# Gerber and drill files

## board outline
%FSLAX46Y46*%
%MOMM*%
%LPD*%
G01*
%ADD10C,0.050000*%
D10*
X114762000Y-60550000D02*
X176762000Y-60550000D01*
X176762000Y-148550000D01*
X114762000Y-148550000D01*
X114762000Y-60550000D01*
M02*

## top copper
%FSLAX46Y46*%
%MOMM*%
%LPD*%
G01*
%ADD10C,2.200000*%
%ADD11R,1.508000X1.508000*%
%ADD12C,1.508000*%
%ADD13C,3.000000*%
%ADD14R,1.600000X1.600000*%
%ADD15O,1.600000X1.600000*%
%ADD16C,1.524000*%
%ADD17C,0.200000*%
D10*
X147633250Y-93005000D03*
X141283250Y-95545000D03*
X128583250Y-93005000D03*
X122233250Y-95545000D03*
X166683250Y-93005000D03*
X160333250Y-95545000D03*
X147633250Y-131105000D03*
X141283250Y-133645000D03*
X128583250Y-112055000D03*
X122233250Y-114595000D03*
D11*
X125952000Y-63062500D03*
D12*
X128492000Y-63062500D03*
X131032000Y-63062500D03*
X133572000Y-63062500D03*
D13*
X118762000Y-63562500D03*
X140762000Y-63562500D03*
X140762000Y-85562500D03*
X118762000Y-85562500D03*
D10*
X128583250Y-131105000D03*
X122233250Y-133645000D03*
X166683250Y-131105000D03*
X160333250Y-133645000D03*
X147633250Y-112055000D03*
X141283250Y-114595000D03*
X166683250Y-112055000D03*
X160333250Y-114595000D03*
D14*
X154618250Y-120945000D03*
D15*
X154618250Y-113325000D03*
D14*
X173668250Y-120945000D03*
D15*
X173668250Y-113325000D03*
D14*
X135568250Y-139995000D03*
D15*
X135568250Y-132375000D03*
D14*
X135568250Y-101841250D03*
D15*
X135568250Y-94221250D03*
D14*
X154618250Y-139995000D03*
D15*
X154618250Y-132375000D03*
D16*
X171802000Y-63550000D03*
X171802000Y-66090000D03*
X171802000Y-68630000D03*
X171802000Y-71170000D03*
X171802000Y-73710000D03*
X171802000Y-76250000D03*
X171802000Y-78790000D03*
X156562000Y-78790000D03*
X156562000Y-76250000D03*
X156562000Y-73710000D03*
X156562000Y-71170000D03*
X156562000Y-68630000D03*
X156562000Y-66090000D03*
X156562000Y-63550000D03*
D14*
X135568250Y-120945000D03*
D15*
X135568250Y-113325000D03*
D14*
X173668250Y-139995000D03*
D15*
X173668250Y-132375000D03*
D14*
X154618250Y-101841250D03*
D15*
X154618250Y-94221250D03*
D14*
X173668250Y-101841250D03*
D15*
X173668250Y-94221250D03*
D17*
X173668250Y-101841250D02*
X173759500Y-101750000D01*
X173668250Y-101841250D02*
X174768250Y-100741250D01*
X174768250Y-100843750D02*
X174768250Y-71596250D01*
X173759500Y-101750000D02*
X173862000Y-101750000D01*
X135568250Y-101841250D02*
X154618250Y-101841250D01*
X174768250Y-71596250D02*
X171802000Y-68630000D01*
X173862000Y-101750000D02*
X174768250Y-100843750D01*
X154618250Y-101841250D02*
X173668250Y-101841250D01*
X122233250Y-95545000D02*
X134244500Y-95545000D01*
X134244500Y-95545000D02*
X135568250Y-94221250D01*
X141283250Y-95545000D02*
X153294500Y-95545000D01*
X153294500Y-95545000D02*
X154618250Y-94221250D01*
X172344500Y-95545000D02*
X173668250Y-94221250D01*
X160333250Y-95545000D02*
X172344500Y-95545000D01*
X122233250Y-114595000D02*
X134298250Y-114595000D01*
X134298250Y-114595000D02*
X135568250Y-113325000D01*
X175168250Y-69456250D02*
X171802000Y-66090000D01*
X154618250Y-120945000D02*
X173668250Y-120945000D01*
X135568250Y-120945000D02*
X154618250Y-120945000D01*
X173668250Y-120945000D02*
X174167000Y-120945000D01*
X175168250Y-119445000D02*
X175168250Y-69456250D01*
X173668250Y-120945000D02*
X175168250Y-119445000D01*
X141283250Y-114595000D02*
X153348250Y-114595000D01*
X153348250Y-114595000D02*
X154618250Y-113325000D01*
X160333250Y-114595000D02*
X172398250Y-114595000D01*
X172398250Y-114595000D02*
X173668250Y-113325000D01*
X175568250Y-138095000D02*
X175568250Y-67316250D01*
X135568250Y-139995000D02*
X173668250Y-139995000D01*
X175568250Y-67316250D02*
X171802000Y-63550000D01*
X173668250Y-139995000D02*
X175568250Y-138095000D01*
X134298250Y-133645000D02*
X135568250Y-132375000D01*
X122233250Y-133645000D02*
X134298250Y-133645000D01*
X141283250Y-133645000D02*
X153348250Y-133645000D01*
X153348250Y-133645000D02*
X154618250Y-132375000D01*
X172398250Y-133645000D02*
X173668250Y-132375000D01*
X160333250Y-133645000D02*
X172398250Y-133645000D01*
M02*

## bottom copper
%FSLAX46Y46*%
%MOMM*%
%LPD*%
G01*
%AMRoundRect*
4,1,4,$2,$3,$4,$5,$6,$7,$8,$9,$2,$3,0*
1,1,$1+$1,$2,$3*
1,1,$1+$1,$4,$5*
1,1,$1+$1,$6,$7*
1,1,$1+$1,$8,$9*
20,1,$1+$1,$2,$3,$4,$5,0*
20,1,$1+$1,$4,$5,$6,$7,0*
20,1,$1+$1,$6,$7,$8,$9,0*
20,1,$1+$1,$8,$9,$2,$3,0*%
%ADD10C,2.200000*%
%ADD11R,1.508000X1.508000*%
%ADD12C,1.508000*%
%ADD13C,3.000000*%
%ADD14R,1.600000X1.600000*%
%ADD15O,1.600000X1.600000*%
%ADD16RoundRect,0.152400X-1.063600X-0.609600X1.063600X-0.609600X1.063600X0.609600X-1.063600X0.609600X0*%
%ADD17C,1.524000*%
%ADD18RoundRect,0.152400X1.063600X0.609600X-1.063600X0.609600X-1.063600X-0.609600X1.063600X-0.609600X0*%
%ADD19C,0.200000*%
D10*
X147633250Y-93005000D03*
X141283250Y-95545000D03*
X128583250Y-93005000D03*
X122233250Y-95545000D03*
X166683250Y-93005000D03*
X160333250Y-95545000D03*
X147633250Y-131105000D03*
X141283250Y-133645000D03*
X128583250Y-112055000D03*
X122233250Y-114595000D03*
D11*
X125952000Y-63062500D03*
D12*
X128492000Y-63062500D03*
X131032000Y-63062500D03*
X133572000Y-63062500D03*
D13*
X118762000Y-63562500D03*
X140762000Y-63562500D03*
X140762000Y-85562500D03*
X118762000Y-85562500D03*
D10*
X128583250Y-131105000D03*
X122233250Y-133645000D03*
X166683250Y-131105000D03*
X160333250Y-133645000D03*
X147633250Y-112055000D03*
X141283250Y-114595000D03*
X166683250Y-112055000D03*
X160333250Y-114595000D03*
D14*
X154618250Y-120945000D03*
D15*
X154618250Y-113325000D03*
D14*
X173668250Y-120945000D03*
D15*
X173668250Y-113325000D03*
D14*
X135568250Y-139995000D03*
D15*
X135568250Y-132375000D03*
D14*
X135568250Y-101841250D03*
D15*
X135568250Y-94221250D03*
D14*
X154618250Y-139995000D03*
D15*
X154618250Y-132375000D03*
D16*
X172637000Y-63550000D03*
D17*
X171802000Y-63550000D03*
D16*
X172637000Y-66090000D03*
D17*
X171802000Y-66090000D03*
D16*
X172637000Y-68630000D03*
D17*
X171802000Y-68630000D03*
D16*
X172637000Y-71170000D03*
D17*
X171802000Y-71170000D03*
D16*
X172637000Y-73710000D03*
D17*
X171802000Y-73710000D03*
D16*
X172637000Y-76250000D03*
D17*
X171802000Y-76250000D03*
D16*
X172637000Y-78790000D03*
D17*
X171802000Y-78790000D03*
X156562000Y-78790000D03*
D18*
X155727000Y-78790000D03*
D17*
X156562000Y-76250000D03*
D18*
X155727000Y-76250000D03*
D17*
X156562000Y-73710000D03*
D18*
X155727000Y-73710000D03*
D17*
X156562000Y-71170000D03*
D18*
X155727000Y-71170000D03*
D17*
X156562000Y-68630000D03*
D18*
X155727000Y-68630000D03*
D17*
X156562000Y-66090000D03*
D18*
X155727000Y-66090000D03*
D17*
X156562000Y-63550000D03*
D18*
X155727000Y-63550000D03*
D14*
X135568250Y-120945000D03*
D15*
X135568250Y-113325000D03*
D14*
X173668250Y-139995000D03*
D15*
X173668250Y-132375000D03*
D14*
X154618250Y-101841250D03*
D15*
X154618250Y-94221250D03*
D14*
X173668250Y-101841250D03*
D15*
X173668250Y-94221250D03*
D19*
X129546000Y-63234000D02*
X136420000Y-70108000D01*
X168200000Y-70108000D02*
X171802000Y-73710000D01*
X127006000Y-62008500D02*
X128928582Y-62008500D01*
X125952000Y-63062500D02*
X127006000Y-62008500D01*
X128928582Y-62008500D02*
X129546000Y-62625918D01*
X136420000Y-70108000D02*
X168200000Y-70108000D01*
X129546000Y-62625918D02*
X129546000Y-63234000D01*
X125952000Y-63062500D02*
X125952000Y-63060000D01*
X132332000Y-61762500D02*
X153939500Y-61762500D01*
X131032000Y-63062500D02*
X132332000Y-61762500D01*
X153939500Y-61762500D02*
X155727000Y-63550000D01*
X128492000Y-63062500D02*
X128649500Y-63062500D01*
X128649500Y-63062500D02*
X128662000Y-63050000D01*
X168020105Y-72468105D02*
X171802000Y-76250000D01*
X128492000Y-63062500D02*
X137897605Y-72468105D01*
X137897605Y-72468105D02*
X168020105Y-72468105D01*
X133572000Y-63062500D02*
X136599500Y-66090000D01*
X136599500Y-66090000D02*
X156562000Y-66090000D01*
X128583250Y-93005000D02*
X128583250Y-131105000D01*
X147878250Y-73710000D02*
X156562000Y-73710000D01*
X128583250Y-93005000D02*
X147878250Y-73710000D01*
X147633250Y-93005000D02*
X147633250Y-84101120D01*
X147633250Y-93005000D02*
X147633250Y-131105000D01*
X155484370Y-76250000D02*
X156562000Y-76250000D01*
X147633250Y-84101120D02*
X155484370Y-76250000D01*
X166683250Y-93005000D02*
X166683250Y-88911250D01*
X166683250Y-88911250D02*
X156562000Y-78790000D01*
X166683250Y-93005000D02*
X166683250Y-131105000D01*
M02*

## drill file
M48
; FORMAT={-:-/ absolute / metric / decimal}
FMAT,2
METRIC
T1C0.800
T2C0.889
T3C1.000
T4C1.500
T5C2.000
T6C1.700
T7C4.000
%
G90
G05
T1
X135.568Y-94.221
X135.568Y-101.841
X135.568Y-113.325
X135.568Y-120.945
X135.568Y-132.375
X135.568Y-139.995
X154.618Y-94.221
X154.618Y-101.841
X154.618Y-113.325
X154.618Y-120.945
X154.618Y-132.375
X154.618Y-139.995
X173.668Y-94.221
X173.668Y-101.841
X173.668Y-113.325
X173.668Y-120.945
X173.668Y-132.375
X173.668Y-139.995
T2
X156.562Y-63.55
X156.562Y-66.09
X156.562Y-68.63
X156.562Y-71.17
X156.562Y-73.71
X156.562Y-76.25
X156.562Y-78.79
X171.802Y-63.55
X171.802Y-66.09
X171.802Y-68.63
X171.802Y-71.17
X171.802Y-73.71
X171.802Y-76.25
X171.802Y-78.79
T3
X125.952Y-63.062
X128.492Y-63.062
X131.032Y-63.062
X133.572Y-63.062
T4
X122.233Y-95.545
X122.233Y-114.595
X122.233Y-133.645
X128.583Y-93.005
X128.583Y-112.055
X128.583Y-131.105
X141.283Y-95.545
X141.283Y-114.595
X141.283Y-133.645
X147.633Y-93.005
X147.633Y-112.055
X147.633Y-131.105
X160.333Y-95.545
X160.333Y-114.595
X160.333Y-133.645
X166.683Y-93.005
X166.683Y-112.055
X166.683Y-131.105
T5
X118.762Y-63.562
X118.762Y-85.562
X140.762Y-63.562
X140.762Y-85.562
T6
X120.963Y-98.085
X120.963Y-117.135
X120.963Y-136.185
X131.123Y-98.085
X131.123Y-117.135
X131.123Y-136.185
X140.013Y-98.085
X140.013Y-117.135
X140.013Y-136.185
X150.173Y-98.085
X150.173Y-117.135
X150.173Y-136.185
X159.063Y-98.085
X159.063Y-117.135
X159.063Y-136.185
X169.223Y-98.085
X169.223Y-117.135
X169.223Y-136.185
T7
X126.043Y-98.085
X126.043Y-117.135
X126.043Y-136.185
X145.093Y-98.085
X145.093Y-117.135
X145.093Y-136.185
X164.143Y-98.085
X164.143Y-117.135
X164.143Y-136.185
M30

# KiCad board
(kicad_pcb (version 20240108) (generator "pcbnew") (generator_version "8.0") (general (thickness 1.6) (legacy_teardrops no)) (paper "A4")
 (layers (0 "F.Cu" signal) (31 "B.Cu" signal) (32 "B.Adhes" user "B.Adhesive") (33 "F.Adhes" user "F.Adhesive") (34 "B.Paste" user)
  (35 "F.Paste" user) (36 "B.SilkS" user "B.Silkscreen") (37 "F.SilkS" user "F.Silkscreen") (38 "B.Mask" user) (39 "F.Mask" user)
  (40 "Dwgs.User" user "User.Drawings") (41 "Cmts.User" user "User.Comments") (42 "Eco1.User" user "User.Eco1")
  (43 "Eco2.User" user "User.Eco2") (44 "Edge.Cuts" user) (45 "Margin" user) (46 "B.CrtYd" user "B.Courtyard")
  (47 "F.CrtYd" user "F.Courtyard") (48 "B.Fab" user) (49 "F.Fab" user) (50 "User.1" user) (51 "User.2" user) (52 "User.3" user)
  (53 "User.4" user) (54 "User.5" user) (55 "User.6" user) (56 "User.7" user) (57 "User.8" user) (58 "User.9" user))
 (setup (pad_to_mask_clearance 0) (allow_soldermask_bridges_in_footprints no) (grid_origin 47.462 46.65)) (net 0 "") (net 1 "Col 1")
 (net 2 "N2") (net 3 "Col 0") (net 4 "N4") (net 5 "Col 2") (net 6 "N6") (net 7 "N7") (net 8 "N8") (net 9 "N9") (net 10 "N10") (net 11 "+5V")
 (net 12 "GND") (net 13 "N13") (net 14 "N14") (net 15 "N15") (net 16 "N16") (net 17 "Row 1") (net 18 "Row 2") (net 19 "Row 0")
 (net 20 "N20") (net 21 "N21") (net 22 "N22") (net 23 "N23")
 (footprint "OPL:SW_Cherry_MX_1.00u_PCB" (layer "F.Cu") (at 147.63325 93.005)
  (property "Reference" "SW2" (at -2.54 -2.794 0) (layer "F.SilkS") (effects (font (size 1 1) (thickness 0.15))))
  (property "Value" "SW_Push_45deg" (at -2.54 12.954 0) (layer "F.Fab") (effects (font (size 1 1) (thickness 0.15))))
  (pad "" np_thru_hole circle (at -7.62 5.08) (size 1.7 1.7) (drill 1.7) (layers "*.Cu" "*.Mask"))
  (pad "" np_thru_hole circle (at -2.54 5.08) (size 4 4) (drill 4) (layers "*.Cu" "*.Mask"))
  (pad "" np_thru_hole circle (at 2.54 5.08) (size 1.7 1.7) (drill 1.7) (layers "*.Cu" "*.Mask"))
  (pad "1" thru_hole circle (at 0 0) (size 2.2 2.2) (drill 1.5) (layers "*.Cu" "*.Mask") (remove_unused_layers no) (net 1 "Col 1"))
  (pad "2" thru_hole circle (at -6.35 2.54) (size 2.2 2.2) (drill 1.5) (layers "*.Cu" "*.Mask") (remove_unused_layers no) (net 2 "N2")))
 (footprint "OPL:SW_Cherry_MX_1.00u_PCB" (layer "F.Cu") (at 128.58325 93.005)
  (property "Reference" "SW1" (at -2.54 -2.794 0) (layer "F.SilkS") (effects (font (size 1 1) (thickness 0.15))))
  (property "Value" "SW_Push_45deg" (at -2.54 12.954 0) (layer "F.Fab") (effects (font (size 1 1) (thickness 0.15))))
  (pad "" np_thru_hole circle (at -7.62 5.08) (size 1.7 1.7) (drill 1.7) (layers "*.Cu" "*.Mask"))
  (pad "" np_thru_hole circle (at -2.54 5.08) (size 4 4) (drill 4) (layers "*.Cu" "*.Mask"))
  (pad "" np_thru_hole circle (at 2.54 5.08) (size 1.7 1.7) (drill 1.7) (layers "*.Cu" "*.Mask"))
  (pad "1" thru_hole circle (at 0 0) (size 2.2 2.2) (drill 1.5) (layers "*.Cu" "*.Mask") (remove_unused_layers no) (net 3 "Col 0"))
  (pad "2" thru_hole circle (at -6.35 2.54) (size 2.2 2.2) (drill 1.5) (layers "*.Cu" "*.Mask") (remove_unused_layers no) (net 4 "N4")))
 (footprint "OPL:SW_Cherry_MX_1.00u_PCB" (layer "F.Cu") (at 166.68325 93.005)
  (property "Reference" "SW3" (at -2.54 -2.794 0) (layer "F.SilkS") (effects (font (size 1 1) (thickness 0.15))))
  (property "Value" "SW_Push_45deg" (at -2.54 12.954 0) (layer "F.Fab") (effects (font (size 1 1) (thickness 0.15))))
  (pad "" np_thru_hole circle (at -7.62 5.08) (size 1.7 1.7) (drill 1.7) (layers "*.Cu" "*.Mask"))
  (pad "" np_thru_hole circle (at -2.54 5.08) (size 4 4) (drill 4) (layers "*.Cu" "*.Mask"))
  (pad "" np_thru_hole circle (at 2.54 5.08) (size 1.7 1.7) (drill 1.7) (layers "*.Cu" "*.Mask"))
  (pad "1" thru_hole circle (at 0 0) (size 2.2 2.2) (drill 1.5) (layers "*.Cu" "*.Mask") (remove_unused_layers no) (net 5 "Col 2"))
  (pad "2" thru_hole circle (at -6.35 2.54) (size 2.2 2.2) (drill 1.5) (layers "*.Cu" "*.Mask") (remove_unused_layers no) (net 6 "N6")))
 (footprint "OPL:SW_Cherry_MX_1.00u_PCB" (layer "F.Cu") (at 147.63325 131.105)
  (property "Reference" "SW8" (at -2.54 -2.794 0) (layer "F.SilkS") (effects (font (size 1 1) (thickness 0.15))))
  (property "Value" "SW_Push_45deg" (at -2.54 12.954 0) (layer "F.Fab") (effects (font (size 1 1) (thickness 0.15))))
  (pad "" np_thru_hole circle (at -7.62 5.08) (size 1.7 1.7) (drill 1.7) (layers "*.Cu" "*.Mask"))
  (pad "" np_thru_hole circle (at -2.54 5.08) (size 4 4) (drill 4) (layers "*.Cu" "*.Mask"))
  (pad "" np_thru_hole circle (at 2.54 5.08) (size 1.7 1.7) (drill 1.7) (layers "*.Cu" "*.Mask"))
  (pad "1" thru_hole circle (at 0 0) (size 2.2 2.2) (drill 1.5) (layers "*.Cu" "*.Mask") (remove_unused_layers no) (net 1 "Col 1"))
  (pad "2" thru_hole circle (at -6.35 2.54) (size 2.2 2.2) (drill 1.5) (layers "*.Cu" "*.Mask") (remove_unused_layers no) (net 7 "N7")))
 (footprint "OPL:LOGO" (layer "F.Cu") (at 161.562 84.85)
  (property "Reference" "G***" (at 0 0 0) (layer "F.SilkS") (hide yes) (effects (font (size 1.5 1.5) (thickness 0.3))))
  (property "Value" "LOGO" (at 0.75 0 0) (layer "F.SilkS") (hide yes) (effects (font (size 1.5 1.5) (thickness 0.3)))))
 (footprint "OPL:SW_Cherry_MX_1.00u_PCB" (layer "F.Cu") (at 128.58325 112.055)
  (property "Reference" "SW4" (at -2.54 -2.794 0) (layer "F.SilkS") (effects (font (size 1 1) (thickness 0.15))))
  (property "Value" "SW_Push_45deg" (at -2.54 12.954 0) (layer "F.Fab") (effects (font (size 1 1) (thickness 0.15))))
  (pad "" np_thru_hole circle (at -7.62 5.08) (size 1.7 1.7) (drill 1.7) (layers "*.Cu" "*.Mask"))
  (pad "" np_thru_hole circle (at -2.54 5.08) (size 4 4) (drill 4) (layers "*.Cu" "*.Mask"))
  (pad "" np_thru_hole circle (at 2.54 5.08) (size 1.7 1.7) (drill 1.7) (layers "*.Cu" "*.Mask"))
  (pad "1" thru_hole circle (at 0 0) (size 2.2 2.2) (drill 1.5) (layers "*.Cu" "*.Mask") (remove_unused_layers no) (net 3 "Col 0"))
  (pad "2" thru_hole circle (at -6.35 2.54) (size 2.2 2.2) (drill 1.5) (layers "*.Cu" "*.Mask") (remove_unused_layers no) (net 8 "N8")))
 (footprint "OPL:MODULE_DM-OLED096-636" (layer "F.Cu") (at 129.762 74.5625)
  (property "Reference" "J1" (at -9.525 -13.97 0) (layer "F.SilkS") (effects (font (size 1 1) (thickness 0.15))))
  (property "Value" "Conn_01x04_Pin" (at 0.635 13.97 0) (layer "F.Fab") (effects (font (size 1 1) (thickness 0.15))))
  (pad "1" thru_hole rect (at -3.81 -11.5) (size 1.508 1.508) (drill 1) (layers "*.Cu" "*.Mask") (remove_unused_layers no) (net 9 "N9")
   (solder_mask_margin 0.102))
  (pad "2" thru_hole circle (at -1.27 -11.5) (size 1.508 1.508) (drill 1) (layers "*.Cu" "*.Mask") (remove_unused_layers no) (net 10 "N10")
   (solder_mask_margin 0.102))
  (pad "3" thru_hole circle (at 1.27 -11.5) (size 1.508 1.508) (drill 1) (layers "*.Cu" "*.Mask") (remove_unused_layers no) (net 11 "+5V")
   (solder_mask_margin 0.102))
  (pad "4" thru_hole circle (at 3.81 -11.5) (size 1.508 1.508) (drill 1) (layers "*.Cu" "*.Mask") (remove_unused_layers no) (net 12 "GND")
   (solder_mask_margin 0.102))
  (pad "S1" thru_hole circle (at -11 -11) (size 3 3) (drill 2) (layers "*.Cu" "*.Mask") (remove_unused_layers no) (solder_mask_margin 0.102))
  (pad "S2" thru_hole circle (at 11 -11) (size 3 3) (drill 2) (layers "*.Cu" "*.Mask") (remove_unused_layers no) (solder_mask_margin 0.102))
  (pad "S3" thru_hole circle (at 11 11) (size 3 3) (drill 2) (layers "*.Cu" "*.Mask") (remove_unused_layers no) (solder_mask_margin 0.102))
  (pad "S4" thru_hole circle (at -11 11) (size 3 3) (drill 2) (layers "*.Cu" "*.Mask") (remove_unused_layers no) (solder_mask_margin 0.102)))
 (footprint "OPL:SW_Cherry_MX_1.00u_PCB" (layer "F.Cu") (at 128.58325 131.105)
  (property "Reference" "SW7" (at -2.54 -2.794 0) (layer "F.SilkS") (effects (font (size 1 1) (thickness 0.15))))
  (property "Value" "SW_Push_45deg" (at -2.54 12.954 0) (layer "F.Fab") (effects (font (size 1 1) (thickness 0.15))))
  (pad "" np_thru_hole circle (at -7.62 5.08) (size 1.7 1.7) (drill 1.7) (layers "*.Cu" "*.Mask"))
  (pad "" np_thru_hole circle (at -2.54 5.08) (size 4 4) (drill 4) (layers "*.Cu" "*.Mask"))
  (pad "" np_thru_hole circle (at 2.54 5.08) (size 1.7 1.7) (drill 1.7) (layers "*.Cu" "*.Mask"))
  (pad "1" thru_hole circle (at 0 0) (size 2.2 2.2) (drill 1.5) (layers "*.Cu" "*.Mask") (remove_unused_layers no) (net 3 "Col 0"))
  (pad "2" thru_hole circle (at -6.35 2.54) (size 2.2 2.2) (drill 1.5) (layers "*.Cu" "*.Mask") (remove_unused_layers no) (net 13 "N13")))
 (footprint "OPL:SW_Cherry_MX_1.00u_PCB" (layer "F.Cu") (at 166.68325 131.105)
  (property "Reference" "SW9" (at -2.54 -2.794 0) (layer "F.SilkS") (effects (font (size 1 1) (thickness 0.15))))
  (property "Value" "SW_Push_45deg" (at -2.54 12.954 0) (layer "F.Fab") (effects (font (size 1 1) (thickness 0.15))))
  (pad "" np_thru_hole circle (at -7.62 5.08) (size 1.7 1.7) (drill 1.7) (layers "*.Cu" "*.Mask"))
  (pad "" np_thru_hole circle (at -2.54 5.08) (size 4 4) (drill 4) (layers "*.Cu" "*.Mask"))
  (pad "" np_thru_hole circle (at 2.54 5.08) (size 1.7 1.7) (drill 1.7) (layers "*.Cu" "*.Mask"))
  (pad "1" thru_hole circle (at 0 0) (size 2.2 2.2) (drill 1.5) (layers "*.Cu" "*.Mask") (remove_unused_layers no) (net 5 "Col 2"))
  (pad "2" thru_hole circle (at -6.35 2.54) (size 2.2 2.2) (drill 1.5) (layers "*.Cu" "*.Mask") (remove_unused_layers no) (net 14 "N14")))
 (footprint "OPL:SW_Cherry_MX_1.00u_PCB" (layer "F.Cu") (at 147.63325 112.055)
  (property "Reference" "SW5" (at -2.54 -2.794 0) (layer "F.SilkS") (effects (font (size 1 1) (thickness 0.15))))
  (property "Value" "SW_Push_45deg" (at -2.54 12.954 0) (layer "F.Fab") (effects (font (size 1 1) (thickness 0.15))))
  (pad "" np_thru_hole circle (at -7.62 5.08) (size 1.7 1.7) (drill 1.7) (layers "*.Cu" "*.Mask"))
  (pad "" np_thru_hole circle (at -2.54 5.08) (size 4 4) (drill 4) (layers "*.Cu" "*.Mask"))
  (pad "" np_thru_hole circle (at 2.54 5.08) (size 1.7 1.7) (drill 1.7) (layers "*.Cu" "*.Mask"))
  (pad "1" thru_hole circle (at 0 0) (size 2.2 2.2) (drill 1.5) (layers "*.Cu" "*.Mask") (remove_unused_layers no) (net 1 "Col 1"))
  (pad "2" thru_hole circle (at -6.35 2.54) (size 2.2 2.2) (drill 1.5) (layers "*.Cu" "*.Mask") (remove_unused_layers no) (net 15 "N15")))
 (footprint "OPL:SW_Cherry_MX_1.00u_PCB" (layer "F.Cu") (at 166.68325 112.055)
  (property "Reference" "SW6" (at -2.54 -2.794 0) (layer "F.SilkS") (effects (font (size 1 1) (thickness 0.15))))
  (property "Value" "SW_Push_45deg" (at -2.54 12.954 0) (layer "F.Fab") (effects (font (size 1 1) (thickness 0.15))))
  (pad "" np_thru_hole circle (at -7.62 5.08) (size 1.7 1.7) (drill 1.7) (layers "*.Cu" "*.Mask"))
  (pad "" np_thru_hole circle (at -2.54 5.08) (size 4 4) (drill 4) (layers "*.Cu" "*.Mask"))
  (pad "" np_thru_hole circle (at 2.54 5.08) (size 1.7 1.7) (drill 1.7) (layers "*.Cu" "*.Mask"))
  (pad "1" thru_hole circle (at 0 0) (size 2.2 2.2) (drill 1.5) (layers "*.Cu" "*.Mask") (remove_unused_layers no) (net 5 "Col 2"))
  (pad "2" thru_hole circle (at -6.35 2.54) (size 2.2 2.2) (drill 1.5) (layers "*.Cu" "*.Mask") (remove_unused_layers no) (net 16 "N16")))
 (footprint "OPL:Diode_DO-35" (layer "B.Cu") (at 154.61825 120.945 90)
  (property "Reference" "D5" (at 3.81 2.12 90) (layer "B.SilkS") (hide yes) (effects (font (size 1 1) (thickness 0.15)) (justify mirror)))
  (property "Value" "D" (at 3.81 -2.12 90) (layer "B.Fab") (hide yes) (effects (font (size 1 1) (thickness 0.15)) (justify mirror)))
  (pad "1" thru_hole rect (at 0 0 90) (size 1.6 1.6) (drill 0.8) (layers "*.Cu" "*.Mask") (remove_unused_layers no) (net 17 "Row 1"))
  (pad "2" thru_hole oval (at 7.62 0 90) (size 1.6 1.6) (drill 0.8) (layers "*.Cu" "*.Mask") (remove_unused_layers no) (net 15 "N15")))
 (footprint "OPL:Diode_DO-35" (layer "B.Cu") (at 173.66825 120.945 90)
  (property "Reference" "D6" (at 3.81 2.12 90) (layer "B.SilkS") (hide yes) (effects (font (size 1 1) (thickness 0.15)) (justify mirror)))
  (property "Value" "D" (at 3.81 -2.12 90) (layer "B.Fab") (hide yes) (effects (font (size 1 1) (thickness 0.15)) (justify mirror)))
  (pad "1" thru_hole rect (at 0 0 90) (size 1.6 1.6) (drill 0.8) (layers "*.Cu" "*.Mask") (remove_unused_layers no) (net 17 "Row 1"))
  (pad "2" thru_hole oval (at 7.62 0 90) (size 1.6 1.6) (drill 0.8) (layers "*.Cu" "*.Mask") (remove_unused_layers no) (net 16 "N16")))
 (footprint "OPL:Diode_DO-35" (layer "B.Cu") (at 135.56825 139.995 90)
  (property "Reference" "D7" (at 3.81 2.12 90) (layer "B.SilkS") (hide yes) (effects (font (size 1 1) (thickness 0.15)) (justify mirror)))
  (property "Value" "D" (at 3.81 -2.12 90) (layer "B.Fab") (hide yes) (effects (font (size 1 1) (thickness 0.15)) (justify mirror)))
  (pad "1" thru_hole rect (at 0 0 90) (size 1.6 1.6) (drill 0.8) (layers "*.Cu" "*.Mask") (remove_unused_layers no) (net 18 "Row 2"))
  (pad "2" thru_hole oval (at 7.62 0 90) (size 1.6 1.6) (drill 0.8) (layers "*.Cu" "*.Mask") (remove_unused_layers no) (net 13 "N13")))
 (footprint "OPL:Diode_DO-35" (layer "B.Cu") (at 135.56825 101.84125 90)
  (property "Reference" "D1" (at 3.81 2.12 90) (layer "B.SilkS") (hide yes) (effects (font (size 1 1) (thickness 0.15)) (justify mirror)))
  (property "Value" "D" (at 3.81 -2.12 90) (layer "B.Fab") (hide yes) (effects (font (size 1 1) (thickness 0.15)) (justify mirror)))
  (pad "1" thru_hole rect (at 0 0 90) (size 1.6 1.6) (drill 0.8) (layers "*.Cu" "*.Mask") (remove_unused_layers no) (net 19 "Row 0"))
  (pad "2" thru_hole oval (at 7.62 0 90) (size 1.6 1.6) (drill 0.8) (layers "*.Cu" "*.Mask") (remove_unused_layers no) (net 4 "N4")))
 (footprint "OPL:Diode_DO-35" (layer "B.Cu") (at 154.61825 139.995 90)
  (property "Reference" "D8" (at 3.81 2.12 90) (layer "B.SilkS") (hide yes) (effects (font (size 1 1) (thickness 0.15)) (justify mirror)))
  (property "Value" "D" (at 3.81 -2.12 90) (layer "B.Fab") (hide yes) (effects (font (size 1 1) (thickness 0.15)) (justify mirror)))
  (pad "1" thru_hole rect (at 0 0 90) (size 1.6 1.6) (drill 0.8) (layers "*.Cu" "*.Mask") (remove_unused_layers no) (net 18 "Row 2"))
  (pad "2" thru_hole oval (at 7.62 0 90) (size 1.6 1.6) (drill 0.8) (layers "*.Cu" "*.Mask") (remove_unused_layers no) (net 7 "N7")))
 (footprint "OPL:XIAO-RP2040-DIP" (layer "B.Cu") (at 164.182 71.17 180)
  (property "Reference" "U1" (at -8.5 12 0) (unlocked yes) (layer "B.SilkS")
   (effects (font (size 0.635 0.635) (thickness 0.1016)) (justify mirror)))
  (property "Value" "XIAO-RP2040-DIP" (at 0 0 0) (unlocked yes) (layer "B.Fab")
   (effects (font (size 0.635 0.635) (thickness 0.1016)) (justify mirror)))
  (pad "1" smd roundrect (at -8.455 7.62) (size 2.432 1.524) (layers "B.Cu" "B.Mask") (roundrect_rratio 0.1) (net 18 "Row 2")
   (thermal_bridge_angle 45))
  (pad "1" thru_hole circle (at -7.62 7.62) (size 1.524 1.524) (drill 0.889) (layers "*.Cu" "*.Mask") (remove_unused_layers no)
   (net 18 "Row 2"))
  (pad "2" smd roundrect (at -8.455 5.08) (size 2.432 1.524) (layers "B.Cu" "B.Mask") (roundrect_rratio 0.1) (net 17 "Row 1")
   (thermal_bridge_angle 45))
  (pad "2" thru_hole circle (at -7.62 5.08) (size 1.524 1.524) (drill 0.889) (layers "*.Cu" "*.Mask") (remove_unused_layers no)
   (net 17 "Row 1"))
  (pad "3" smd roundrect (at -8.455 2.54) (size 2.432 1.524) (layers "B.Cu" "B.Mask") (roundrect_rratio 0.1) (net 19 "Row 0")
   (thermal_bridge_angle 45))
  (pad "3" thru_hole circle (at -7.62 2.54) (size 1.524 1.524) (drill 0.889) (layers "*.Cu" "*.Mask") (remove_unused_layers no)
   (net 19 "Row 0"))
  (pad "4" smd roundrect (at -8.455 0) (size 2.432 1.524) (layers "B.Cu" "B.Mask") (roundrect_rratio 0.1) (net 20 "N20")
   (thermal_bridge_angle 45))
  (pad "4" thru_hole circle (at -7.62 0) (size 1.524 1.524) (drill 0.889) (layers "*.Cu" "*.Mask") (remove_unused_layers no) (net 20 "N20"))
  (pad "5" smd roundrect (at -8.455 -2.54) (size 2.432 1.524) (layers "B.Cu" "B.Mask") (roundrect_rratio 0.1) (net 9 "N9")
   (thermal_bridge_angle 45))
  (pad "5" thru_hole circle (at -7.62 -2.54) (size 1.524 1.524) (drill 0.889) (layers "*.Cu" "*.Mask") (remove_unused_layers no)
   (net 9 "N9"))
  (pad "6" smd roundrect (at -8.455 -5.08) (size 2.432 1.524) (layers "B.Cu" "B.Mask") (roundrect_rratio 0.1) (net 10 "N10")
   (thermal_bridge_angle 45))
  (pad "6" thru_hole circle (at -7.62 -5.08) (size 1.524 1.524) (drill 0.889) (layers "*.Cu" "*.Mask") (remove_unused_layers no)
   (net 10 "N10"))
  (pad "7" smd roundrect (at -8.455 -7.62) (size 2.432 1.524) (layers "B.Cu" "B.Mask") (roundrect_rratio 0.1) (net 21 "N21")
   (thermal_bridge_angle 45))
  (pad "7" thru_hole circle (at -7.62 -7.62) (size 1.524 1.524) (drill 0.889) (layers "*.Cu" "*.Mask") (remove_unused_layers no)
   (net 21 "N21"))
  (pad "8" thru_hole circle (at 7.62 -7.62 180) (size 1.524 1.524) (drill 0.889) (layers "*.Cu" "*.Mask") (remove_unused_layers no)
   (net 5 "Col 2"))
  (pad "8" smd roundrect (at 8.455 -7.62 180) (size 2.432 1.524) (layers "B.Cu" "B.Mask") (roundrect_rratio 0.1) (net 5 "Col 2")
   (thermal_bridge_angle 45))
  (pad "9" thru_hole circle (at 7.62 -5.08 180) (size 1.524 1.524) (drill 0.889) (layers "*.Cu" "*.Mask") (remove_unused_layers no)
   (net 1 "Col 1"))
  (pad "9" smd roundrect (at 8.455 -5.08 180) (size 2.432 1.524) (layers "B.Cu" "B.Mask") (roundrect_rratio 0.1) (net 1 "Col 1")
   (thermal_bridge_angle 45))
  (pad "10" thru_hole circle (at 7.62 -2.54 180) (size 1.524 1.524) (drill 0.889) (layers "*.Cu" "*.Mask") (remove_unused_layers no)
   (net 3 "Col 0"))
  (pad "10" smd roundrect (at 8.455 -2.54 180) (size 2.432 1.524) (layers "B.Cu" "B.Mask") (roundrect_rratio 0.1) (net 3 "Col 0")
   (thermal_bridge_angle 45))
  (pad "11" thru_hole circle (at 7.62 0 180) (size 1.524 1.524) (drill 0.889) (layers "*.Cu" "*.Mask") (remove_unused_layers no)
   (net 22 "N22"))
  (pad "11" smd roundrect (at 8.455 0 180) (size 2.432 1.524) (layers "B.Cu" "B.Mask") (roundrect_rratio 0.1) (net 22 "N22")
   (thermal_bridge_angle 45))
  (pad "12" thru_hole circle (at 7.62 2.54 180) (size 1.524 1.524) (drill 0.889) (layers "*.Cu" "*.Mask") (remove_unused_layers no)
   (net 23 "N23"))
  (pad "12" smd roundrect (at 8.455 2.54 180) (size 2.432 1.524) (layers "B.Cu" "B.Mask") (roundrect_rratio 0.1) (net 23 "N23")
   (thermal_bridge_angle 45))
  (pad "13" thru_hole circle (at 7.62 5.08 180) (size 1.524 1.524) (drill 0.889) (layers "*.Cu" "*.Mask") (remove_unused_layers no)
   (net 12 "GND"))
  (pad "13" smd roundrect (at 8.455 5.08 180) (size 2.432 1.524) (layers "B.Cu" "B.Mask") (roundrect_rratio 0.1) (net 12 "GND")
   (thermal_bridge_angle 45))
  (pad "14" thru_hole circle (at 7.62 7.62 180) (size 1.524 1.524) (drill 0.889) (layers "*.Cu" "*.Mask") (remove_unused_layers no)
   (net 11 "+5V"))
  (pad "14" smd roundrect (at 8.455 7.62 180) (size 2.432 1.524) (layers "B.Cu" "B.Mask") (roundrect_rratio 0.1) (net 11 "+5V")
   (thermal_bridge_angle 45)))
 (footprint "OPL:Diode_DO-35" (layer "B.Cu") (at 135.56825 120.945 90)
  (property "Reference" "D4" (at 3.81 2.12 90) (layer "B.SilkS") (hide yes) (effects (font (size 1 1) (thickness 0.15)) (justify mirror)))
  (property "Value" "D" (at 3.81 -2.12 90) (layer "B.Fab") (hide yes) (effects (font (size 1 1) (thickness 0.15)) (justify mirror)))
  (pad "1" thru_hole rect (at 0 0 90) (size 1.6 1.6) (drill 0.8) (layers "*.Cu" "*.Mask") (remove_unused_layers no) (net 17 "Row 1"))
  (pad "2" thru_hole oval (at 7.62 0 90) (size 1.6 1.6) (drill 0.8) (layers "*.Cu" "*.Mask") (remove_unused_layers no) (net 8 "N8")))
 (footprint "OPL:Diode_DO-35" (layer "B.Cu") (at 173.66825 139.995 90)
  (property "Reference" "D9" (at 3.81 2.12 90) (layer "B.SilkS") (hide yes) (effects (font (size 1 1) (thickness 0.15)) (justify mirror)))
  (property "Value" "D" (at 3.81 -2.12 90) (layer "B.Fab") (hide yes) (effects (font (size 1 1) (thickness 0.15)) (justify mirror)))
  (pad "1" thru_hole rect (at 0 0 90) (size 1.6 1.6) (drill 0.8) (layers "*.Cu" "*.Mask") (remove_unused_layers no) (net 18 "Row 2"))
  (pad "2" thru_hole oval (at 7.62 0 90) (size 1.6 1.6) (drill 0.8) (layers "*.Cu" "*.Mask") (remove_unused_layers no) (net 14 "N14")))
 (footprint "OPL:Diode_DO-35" (layer "B.Cu") (at 154.61825 101.84125 90)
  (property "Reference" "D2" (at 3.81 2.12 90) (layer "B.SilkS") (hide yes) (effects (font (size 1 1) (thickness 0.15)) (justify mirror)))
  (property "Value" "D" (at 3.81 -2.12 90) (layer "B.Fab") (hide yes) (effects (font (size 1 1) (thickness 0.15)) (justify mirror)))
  (pad "1" thru_hole rect (at 0 0 90) (size 1.6 1.6) (drill 0.8) (layers "*.Cu" "*.Mask") (remove_unused_layers no) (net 19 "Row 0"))
  (pad "2" thru_hole oval (at 7.62 0 90) (size 1.6 1.6) (drill 0.8) (layers "*.Cu" "*.Mask") (remove_unused_layers no) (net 2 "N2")))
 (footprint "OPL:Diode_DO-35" (layer "B.Cu") (at 173.66825 101.84125 90)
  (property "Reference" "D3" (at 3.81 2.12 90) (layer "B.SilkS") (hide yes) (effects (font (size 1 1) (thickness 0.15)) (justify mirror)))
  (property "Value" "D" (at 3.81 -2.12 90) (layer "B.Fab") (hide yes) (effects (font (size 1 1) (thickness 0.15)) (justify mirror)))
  (pad "1" thru_hole rect (at 0 0 90) (size 1.6 1.6) (drill 0.8) (layers "*.Cu" "*.Mask") (remove_unused_layers no) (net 19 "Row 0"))
  (pad "2" thru_hole oval (at 7.62 0 90) (size 1.6 1.6) (drill 0.8) (layers "*.Cu" "*.Mask") (remove_unused_layers no) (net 6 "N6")))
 (gr_rect (start 114.762 60.55) (end 176.762 148.55) (stroke (width 0.05) (type default)) (fill none) (layer "Edge.Cuts"))
 (segment (start 173.66825 101.84125) (end 173.7595 101.75) (width 0.2) (layer "F.Cu") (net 19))
 (segment (start 173.66825 101.84125) (end 174.76825 100.74125) (width 0.2) (layer "F.Cu") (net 19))
 (segment (start 174.76825 100.84375) (end 174.76825 71.59625) (width 0.2) (layer "F.Cu") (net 19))
 (segment (start 173.7595 101.75) (end 173.862 101.75) (width 0.2) (layer "F.Cu") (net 19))
 (segment (start 135.56825 101.84125) (end 154.61825 101.84125) (width 0.2) (layer "F.Cu") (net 19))
 (segment (start 174.76825 71.59625) (end 171.802 68.63) (width 0.2) (layer "F.Cu") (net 19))
 (segment (start 173.862 101.75) (end 174.76825 100.84375) (width 0.2) (layer "F.Cu") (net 19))
 (segment (start 154.61825 101.84125) (end 173.66825 101.84125) (width 0.2) (layer "F.Cu") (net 19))
 (segment (start 122.23325 95.545) (end 134.2445 95.545) (width 0.2) (layer "F.Cu") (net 4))
 (segment (start 134.2445 95.545) (end 135.56825 94.22125) (width 0.2) (layer "F.Cu") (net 4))
 (segment (start 141.28325 95.545) (end 153.2945 95.545) (width 0.2) (layer "F.Cu") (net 2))
 (segment (start 153.2945 95.545) (end 154.61825 94.22125) (width 0.2) (layer "F.Cu") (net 2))
 (segment (start 172.3445 95.545) (end 173.66825 94.22125) (width 0.2) (layer "F.Cu") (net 6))
 (segment (start 160.33325 95.545) (end 172.3445 95.545) (width 0.2) (layer "F.Cu") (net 6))
 (segment (start 122.23325 114.595) (end 134.29825 114.595) (width 0.2) (layer "F.Cu") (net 8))
 (segment (start 134.29825 114.595) (end 135.56825 113.325) (width 0.2) (layer "F.Cu") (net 8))
 (segment (start 175.16825 69.45625) (end 171.802 66.09) (width 0.2) (layer "F.Cu") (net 17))
 (segment (start 154.61825 120.945) (end 173.66825 120.945) (width 0.2) (layer "F.Cu") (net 17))
 (segment (start 135.56825 120.945) (end 154.61825 120.945) (width 0.2) (layer "F.Cu") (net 17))
 (segment (start 173.66825 120.945) (end 174.167 120.945) (width 0.2) (layer "F.Cu") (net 17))
 (segment (start 175.16825 119.445) (end 175.16825 69.45625) (width 0.2) (layer "F.Cu") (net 17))
 (segment (start 173.66825 120.945) (end 175.16825 119.445) (width 0.2) (layer "F.Cu") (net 17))
 (segment (start 141.28325 114.595) (end 153.34825 114.595) (width 0.2) (layer "F.Cu") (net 15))
 (segment (start 153.34825 114.595) (end 154.61825 113.325) (width 0.2) (layer "F.Cu") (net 15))
 (segment (start 160.33325 114.595) (end 172.39825 114.595) (width 0.2) (layer "F.Cu") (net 16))
 (segment (start 172.39825 114.595) (end 173.66825 113.325) (width 0.2) (layer "F.Cu") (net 16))
 (segment (start 175.56825 138.095) (end 175.56825 67.31625) (width 0.2) (layer "F.Cu") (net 18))
 (segment (start 135.56825 139.995) (end 173.66825 139.995) (width 0.2) (layer "F.Cu") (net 18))
 (segment (start 175.56825 67.31625) (end 171.802 63.55) (width 0.2) (layer "F.Cu") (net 18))
 (segment (start 173.66825 139.995) (end 175.56825 138.095) (width 0.2) (layer "F.Cu") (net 18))
 (segment (start 134.29825 133.645) (end 135.56825 132.375) (width 0.2) (layer "F.Cu") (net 13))
 (segment (start 122.23325 133.645) (end 134.29825 133.645) (width 0.2) (layer "F.Cu") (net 13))
 (segment (start 141.28325 133.645) (end 153.34825 133.645) (width 0.2) (layer "F.Cu") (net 7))
 (segment (start 153.34825 133.645) (end 154.61825 132.375) (width 0.2) (layer "F.Cu") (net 7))
 (segment (start 172.39825 133.645) (end 173.66825 132.375) (width 0.2) (layer "F.Cu") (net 14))
 (segment (start 160.33325 133.645) (end 172.39825 133.645) (width 0.2) (layer "F.Cu") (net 14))
 (segment (start 129.546 63.234) (end 136.42 70.108) (width 0.2) (layer "B.Cu") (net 9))
 (segment (start 168.2 70.108) (end 171.802 73.71) (width 0.2) (layer "B.Cu") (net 9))
 (segment (start 127.006 62.0085) (end 128.928582 62.0085) (width 0.2) (layer "B.Cu") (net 9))
 (segment (start 125.952 63.0625) (end 127.006 62.0085) (width 0.2) (layer "B.Cu") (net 9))
 (segment (start 128.928582 62.0085) (end 129.546 62.625918) (width 0.2) (layer "B.Cu") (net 9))
 (segment (start 136.42 70.108) (end 168.2 70.108) (width 0.2) (layer "B.Cu") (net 9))
 (segment (start 129.546 62.625918) (end 129.546 63.234) (width 0.2) (layer "B.Cu") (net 9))
 (segment (start 125.952 63.0625) (end 125.952 63.06) (width 0.2) (layer "B.Cu") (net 9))
 (segment (start 132.332 61.7625) (end 153.9395 61.7625) (width 0.2) (layer "B.Cu") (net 11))
 (segment (start 131.032 63.0625) (end 132.332 61.7625) (width 0.2) (layer "B.Cu") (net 11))
 (segment (start 153.9395 61.7625) (end 155.727 63.55) (width 0.2) (layer "B.Cu") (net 11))
 (segment (start 128.492 63.0625) (end 128.6495 63.0625) (width 0.2) (layer "B.Cu") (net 10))
 (segment (start 128.6495 63.0625) (end 128.662 63.05) (width 0.2) (layer "B.Cu") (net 10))
 (segment (start 168.020105 72.468105) (end 171.802 76.25) (width 0.2) (layer "B.Cu") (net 10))
 (segment (start 128.492 63.0625) (end 137.897605 72.468105) (width 0.2) (layer "B.Cu") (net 10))
 (segment (start 137.897605 72.468105) (end 168.020105 72.468105) (width 0.2) (layer "B.Cu") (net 10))
 (segment (start 133.572 63.0625) (end 136.5995 66.09) (width 0.2) (layer "B.Cu") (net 12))
 (segment (start 136.5995 66.09) (end 156.562 66.09) (width 0.2) (layer "B.Cu") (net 12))
 (segment (start 128.58325 93.005) (end 128.58325 131.105) (width 0.2) (layer "B.Cu") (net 3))
 (segment (start 147.87825 73.71) (end 156.562 73.71) (width 0.2) (layer "B.Cu") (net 3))
 (segment (start 128.58325 93.005) (end 147.87825 73.71) (width 0.2) (layer "B.Cu") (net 3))
 (segment (start 147.63325 93.005) (end 147.63325 84.10112) (width 0.2) (layer "B.Cu") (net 1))
 (segment (start 147.63325 93.005) (end 147.63325 131.105) (width 0.2) (layer "B.Cu") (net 1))
 (segment (start 155.48437 76.25) (end 156.562 76.25) (width 0.2) (layer "B.Cu") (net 1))
 (segment (start 147.63325 84.10112) (end 155.48437 76.25) (width 0.2) (layer "B.Cu") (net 1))
 (segment (start 166.68325 93.005) (end 166.68325 88.91125) (width 0.2) (layer "B.Cu") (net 5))
 (segment (start 166.68325 88.91125) (end 156.562 78.79) (width 0.2) (layer "B.Cu") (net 5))
 (segment (start 166.68325 93.005) (end 166.68325 131.105) (width 0.2) (layer "B.Cu") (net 5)))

